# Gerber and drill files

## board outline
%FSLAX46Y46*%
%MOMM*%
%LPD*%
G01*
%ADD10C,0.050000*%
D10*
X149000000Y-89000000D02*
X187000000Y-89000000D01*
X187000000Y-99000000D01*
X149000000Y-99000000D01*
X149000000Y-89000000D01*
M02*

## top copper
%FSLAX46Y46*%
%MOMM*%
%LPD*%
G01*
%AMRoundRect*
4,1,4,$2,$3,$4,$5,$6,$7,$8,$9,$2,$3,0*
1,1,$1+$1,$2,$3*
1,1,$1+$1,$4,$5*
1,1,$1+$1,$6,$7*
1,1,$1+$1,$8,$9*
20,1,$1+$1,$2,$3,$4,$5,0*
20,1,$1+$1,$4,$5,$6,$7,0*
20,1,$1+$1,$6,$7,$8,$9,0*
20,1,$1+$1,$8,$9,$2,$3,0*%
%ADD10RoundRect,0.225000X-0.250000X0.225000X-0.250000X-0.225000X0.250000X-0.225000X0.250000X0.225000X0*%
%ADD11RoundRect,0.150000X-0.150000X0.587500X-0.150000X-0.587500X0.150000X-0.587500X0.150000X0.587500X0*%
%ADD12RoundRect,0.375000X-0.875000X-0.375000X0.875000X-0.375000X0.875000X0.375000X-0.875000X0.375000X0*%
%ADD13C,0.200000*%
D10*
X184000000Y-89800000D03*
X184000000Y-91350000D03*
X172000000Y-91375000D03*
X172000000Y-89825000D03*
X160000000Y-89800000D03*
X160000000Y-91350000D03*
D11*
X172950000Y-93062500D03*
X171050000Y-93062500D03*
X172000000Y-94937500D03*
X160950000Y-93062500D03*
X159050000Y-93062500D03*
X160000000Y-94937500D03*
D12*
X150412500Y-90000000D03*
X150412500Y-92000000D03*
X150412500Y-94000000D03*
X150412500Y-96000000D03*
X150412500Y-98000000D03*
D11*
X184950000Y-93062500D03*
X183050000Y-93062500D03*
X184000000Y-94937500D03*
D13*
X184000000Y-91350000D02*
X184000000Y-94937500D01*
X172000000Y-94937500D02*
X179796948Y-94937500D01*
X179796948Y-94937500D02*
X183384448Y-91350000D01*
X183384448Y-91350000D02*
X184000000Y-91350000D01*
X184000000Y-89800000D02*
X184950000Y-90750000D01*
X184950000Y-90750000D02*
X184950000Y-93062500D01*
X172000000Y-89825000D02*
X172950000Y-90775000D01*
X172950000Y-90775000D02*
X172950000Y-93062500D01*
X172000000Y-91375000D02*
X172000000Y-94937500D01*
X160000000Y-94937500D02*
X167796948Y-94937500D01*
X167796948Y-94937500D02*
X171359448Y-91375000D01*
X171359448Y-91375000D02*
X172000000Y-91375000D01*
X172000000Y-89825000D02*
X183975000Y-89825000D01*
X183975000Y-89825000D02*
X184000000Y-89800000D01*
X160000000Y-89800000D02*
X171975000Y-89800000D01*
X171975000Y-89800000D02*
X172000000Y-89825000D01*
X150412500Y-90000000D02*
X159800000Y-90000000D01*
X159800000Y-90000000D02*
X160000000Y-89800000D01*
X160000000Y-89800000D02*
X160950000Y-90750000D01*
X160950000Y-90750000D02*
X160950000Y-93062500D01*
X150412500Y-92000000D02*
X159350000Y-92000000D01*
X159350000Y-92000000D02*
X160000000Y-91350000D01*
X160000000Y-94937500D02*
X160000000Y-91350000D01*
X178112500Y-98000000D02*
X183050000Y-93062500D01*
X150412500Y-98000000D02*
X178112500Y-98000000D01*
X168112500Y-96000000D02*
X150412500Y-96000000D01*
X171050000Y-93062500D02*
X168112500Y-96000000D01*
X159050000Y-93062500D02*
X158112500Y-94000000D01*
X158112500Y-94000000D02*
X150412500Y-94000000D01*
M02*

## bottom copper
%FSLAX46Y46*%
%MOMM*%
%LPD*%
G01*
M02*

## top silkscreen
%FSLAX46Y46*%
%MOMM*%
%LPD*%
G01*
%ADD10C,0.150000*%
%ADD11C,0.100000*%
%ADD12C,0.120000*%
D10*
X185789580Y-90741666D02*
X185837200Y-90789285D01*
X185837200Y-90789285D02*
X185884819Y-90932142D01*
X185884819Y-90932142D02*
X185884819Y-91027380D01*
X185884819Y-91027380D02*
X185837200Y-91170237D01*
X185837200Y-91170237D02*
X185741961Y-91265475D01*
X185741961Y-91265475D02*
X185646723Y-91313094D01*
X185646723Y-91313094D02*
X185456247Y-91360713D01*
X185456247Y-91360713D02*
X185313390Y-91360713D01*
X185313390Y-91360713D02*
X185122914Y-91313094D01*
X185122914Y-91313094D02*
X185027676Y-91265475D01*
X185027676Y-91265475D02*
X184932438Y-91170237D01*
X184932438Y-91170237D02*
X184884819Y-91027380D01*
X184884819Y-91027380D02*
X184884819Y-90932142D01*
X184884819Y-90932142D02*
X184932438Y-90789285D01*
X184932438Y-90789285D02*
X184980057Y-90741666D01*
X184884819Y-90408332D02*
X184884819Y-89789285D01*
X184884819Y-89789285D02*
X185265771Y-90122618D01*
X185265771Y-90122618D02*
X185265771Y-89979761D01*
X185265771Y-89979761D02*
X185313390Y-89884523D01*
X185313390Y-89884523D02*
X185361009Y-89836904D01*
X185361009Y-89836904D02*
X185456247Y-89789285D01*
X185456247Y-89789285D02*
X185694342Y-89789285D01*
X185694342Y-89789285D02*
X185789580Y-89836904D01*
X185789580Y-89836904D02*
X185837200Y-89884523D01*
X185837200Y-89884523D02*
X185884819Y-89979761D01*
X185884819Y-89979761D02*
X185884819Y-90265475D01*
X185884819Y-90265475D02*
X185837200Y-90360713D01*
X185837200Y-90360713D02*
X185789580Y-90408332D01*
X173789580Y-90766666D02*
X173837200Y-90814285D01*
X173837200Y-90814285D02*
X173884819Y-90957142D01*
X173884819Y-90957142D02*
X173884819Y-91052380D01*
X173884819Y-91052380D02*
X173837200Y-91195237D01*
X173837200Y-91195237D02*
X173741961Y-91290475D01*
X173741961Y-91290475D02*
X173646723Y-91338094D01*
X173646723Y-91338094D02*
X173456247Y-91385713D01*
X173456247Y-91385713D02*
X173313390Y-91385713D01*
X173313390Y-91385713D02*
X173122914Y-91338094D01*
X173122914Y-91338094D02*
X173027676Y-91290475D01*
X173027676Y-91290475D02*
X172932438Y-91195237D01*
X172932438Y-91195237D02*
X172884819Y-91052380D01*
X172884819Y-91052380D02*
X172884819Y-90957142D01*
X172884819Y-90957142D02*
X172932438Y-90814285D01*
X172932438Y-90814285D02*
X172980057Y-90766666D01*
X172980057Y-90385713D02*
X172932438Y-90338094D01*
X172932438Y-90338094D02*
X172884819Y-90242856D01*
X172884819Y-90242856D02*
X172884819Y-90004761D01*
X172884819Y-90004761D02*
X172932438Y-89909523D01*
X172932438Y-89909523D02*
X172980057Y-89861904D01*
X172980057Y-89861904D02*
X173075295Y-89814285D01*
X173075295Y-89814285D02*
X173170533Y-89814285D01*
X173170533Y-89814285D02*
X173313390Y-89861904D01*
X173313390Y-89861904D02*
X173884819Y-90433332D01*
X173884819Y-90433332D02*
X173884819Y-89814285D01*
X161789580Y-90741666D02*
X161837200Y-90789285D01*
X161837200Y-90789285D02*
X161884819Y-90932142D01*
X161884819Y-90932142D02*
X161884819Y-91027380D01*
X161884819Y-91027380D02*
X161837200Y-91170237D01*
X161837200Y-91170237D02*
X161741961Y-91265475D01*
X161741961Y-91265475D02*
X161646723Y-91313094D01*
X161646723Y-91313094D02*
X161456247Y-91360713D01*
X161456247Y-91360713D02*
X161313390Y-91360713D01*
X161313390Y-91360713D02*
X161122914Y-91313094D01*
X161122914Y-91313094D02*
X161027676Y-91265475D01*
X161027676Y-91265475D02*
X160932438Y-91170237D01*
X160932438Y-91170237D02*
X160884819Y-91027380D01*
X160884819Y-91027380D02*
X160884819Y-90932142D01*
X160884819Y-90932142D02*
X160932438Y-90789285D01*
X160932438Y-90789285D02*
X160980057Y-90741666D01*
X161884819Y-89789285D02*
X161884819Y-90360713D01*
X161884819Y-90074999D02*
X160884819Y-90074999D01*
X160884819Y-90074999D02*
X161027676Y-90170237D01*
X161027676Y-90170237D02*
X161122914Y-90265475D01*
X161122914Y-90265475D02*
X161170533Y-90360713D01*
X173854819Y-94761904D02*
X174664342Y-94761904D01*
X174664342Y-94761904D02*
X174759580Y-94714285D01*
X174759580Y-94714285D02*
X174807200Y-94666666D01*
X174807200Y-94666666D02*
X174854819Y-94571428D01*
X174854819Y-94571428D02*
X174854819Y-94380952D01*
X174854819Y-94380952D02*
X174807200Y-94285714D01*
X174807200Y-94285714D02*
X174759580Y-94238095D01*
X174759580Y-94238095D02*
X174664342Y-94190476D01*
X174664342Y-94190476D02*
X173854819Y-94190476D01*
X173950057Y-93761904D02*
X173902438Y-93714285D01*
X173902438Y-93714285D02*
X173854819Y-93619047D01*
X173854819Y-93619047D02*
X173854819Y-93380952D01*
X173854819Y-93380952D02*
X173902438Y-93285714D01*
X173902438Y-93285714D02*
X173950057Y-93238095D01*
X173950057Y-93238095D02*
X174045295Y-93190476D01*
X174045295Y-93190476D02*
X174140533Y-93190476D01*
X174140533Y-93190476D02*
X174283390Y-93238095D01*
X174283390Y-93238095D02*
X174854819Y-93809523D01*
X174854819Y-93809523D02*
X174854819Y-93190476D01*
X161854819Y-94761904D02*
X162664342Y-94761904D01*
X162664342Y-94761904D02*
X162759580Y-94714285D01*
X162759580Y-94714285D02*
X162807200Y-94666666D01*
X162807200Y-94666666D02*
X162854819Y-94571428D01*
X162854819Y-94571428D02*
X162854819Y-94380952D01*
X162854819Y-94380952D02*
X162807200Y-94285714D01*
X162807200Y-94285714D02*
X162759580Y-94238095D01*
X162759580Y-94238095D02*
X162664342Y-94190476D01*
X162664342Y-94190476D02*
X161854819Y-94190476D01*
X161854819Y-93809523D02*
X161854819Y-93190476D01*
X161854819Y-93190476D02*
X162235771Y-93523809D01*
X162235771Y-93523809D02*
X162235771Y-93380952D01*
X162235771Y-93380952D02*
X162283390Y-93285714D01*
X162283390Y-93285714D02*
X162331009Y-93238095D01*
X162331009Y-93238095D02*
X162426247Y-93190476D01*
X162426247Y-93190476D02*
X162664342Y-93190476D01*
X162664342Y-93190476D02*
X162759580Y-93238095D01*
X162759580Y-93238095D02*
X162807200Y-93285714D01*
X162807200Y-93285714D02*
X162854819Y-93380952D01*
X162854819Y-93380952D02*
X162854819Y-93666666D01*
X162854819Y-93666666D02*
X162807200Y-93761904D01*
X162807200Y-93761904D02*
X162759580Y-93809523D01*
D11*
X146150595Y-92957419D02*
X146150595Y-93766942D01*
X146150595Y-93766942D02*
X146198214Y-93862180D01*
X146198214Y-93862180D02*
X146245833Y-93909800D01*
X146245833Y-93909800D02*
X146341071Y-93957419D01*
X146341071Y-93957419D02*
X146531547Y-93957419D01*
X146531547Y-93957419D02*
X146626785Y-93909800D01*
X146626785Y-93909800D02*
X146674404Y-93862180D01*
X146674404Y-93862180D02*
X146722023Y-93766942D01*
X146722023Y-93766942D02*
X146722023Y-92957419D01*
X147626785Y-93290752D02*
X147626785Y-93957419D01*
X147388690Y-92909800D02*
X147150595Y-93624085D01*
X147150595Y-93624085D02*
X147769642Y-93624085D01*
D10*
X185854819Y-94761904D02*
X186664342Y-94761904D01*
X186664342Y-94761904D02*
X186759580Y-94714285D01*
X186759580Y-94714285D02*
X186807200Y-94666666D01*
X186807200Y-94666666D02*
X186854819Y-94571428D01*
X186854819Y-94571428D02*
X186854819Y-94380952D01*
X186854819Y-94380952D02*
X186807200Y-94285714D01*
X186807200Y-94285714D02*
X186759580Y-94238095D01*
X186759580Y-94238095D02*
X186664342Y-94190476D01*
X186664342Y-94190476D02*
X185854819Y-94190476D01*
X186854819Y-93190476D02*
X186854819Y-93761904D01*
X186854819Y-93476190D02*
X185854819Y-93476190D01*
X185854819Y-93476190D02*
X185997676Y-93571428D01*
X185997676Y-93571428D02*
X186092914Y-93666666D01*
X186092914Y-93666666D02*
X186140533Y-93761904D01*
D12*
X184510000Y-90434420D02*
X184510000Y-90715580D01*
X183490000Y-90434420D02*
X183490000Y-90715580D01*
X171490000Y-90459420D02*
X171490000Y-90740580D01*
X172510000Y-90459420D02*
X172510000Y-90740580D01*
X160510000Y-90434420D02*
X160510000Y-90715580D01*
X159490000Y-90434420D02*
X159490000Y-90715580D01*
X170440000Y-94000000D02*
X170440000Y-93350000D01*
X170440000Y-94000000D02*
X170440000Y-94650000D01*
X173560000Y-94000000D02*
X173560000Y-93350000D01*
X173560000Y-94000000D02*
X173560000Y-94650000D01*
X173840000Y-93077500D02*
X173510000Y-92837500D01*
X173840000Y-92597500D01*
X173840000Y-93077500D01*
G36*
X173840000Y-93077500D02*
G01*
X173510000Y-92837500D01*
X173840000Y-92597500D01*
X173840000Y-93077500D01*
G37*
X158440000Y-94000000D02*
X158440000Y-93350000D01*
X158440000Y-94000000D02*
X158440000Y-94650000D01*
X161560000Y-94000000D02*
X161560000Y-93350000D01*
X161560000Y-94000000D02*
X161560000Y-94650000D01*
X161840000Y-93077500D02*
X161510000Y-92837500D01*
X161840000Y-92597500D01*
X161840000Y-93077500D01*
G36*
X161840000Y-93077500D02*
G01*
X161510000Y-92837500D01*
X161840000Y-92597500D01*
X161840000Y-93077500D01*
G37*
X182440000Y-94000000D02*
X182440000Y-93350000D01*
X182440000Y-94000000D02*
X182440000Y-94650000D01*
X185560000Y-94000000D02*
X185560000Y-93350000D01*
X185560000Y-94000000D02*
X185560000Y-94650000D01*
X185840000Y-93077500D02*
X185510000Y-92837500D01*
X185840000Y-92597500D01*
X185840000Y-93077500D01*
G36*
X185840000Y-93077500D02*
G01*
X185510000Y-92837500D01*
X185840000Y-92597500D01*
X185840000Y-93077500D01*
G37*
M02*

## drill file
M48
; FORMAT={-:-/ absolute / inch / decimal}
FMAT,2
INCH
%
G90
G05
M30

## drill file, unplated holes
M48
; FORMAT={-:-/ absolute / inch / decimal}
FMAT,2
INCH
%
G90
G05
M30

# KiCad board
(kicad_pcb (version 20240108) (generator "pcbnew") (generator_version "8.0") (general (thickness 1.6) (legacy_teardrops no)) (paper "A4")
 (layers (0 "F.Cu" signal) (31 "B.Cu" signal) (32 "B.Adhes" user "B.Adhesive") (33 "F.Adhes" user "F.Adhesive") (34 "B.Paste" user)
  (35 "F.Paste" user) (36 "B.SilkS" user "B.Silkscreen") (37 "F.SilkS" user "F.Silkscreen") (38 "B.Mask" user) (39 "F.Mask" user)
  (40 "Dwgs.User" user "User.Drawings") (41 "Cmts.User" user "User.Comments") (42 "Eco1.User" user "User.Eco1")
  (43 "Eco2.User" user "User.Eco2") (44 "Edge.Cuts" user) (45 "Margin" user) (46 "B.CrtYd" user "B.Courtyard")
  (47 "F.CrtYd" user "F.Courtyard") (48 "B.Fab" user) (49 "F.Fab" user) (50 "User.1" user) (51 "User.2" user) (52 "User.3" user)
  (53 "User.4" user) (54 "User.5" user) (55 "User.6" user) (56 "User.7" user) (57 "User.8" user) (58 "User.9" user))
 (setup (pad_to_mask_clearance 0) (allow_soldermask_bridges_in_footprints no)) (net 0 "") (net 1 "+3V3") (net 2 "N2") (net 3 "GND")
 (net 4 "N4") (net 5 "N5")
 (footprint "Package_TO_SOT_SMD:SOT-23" (layer "F.Cu") (at 172 94 -90)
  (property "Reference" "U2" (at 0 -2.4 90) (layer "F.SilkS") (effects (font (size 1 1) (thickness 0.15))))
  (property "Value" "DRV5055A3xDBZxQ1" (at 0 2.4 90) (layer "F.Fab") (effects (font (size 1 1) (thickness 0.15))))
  (fp_line (start 0 1.56) (end -0.65 1.56) (stroke (width 0.12) (type solid)) (layer "F.SilkS"))
  (fp_line (start 0 1.56) (end 0.65 1.56) (stroke (width 0.12) (type solid)) (layer "F.SilkS"))
  (fp_line (start 0 -1.56) (end -0.65 -1.56) (stroke (width 0.12) (type solid)) (layer "F.SilkS"))
  (fp_line (start 0 -1.56) (end 0.65 -1.56) (stroke (width 0.12) (type solid)) (layer "F.SilkS"))
  (fp_poly
   (pts (xy -1.1625 -1.51) (xy -1.4025 -1.84) (xy -0.9225 -1.84) (xy -1.1625 -1.51)) (stroke (width 0.12) (type solid)) (fill solid)
   (layer "F.SilkS"))
  (pad "1" smd roundrect (at -0.9375 -0.95 270) (size 1.475 0.6) (layers "F.Cu" "F.Paste" "F.Mask") (roundrect_rratio 0.25) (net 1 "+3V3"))
  (pad "2" smd roundrect (at -0.9375 0.95 270) (size 1.475 0.6) (layers "F.Cu" "F.Paste" "F.Mask") (roundrect_rratio 0.25) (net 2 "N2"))
  (pad "3" smd roundrect (at 0.9375 0 270) (size 1.475 0.6) (layers "F.Cu" "F.Paste" "F.Mask") (roundrect_rratio 0.25) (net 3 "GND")))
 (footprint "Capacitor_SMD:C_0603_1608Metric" (layer "F.Cu") (at 184 90.575 -90)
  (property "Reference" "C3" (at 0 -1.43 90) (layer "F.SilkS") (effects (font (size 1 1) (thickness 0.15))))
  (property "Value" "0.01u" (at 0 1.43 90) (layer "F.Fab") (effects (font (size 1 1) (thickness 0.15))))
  (fp_line (start -0.14058 0.51) (end 0.14058 0.51) (stroke (width 0.12) (type solid)) (layer "F.SilkS"))
  (fp_line (start -0.14058 -0.51) (end 0.14058 -0.51) (stroke (width 0.12) (type solid)) (layer "F.SilkS"))
  (pad "1" smd roundrect (at -0.775 0 270) (size 0.9 0.95) (layers "F.Cu" "F.Paste" "F.Mask") (roundrect_rratio 0.25) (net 1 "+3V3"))
  (pad "2" smd roundrect (at 0.775 0 270) (size 0.9 0.95) (layers "F.Cu" "F.Paste" "F.Mask") (roundrect_rratio 0.25) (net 3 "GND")))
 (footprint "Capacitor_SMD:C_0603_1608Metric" (layer "F.Cu") (at 160 90.575 -90)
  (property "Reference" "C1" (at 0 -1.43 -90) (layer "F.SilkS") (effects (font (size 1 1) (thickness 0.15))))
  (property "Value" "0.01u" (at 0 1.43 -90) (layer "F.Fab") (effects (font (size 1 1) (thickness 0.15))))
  (fp_line (start -0.14058 0.51) (end 0.14058 0.51) (stroke (width 0.12) (type solid)) (layer "F.SilkS"))
  (fp_line (start -0.14058 -0.51) (end 0.14058 -0.51) (stroke (width 0.12) (type solid)) (layer "F.SilkS"))
  (pad "1" smd roundrect (at -0.775 0 270) (size 0.9 0.95) (layers "F.Cu" "F.Paste" "F.Mask") (roundrect_rratio 0.25) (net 1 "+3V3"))
  (pad "2" smd roundrect (at 0.775 0 270) (size 0.9 0.95) (layers "F.Cu" "F.Paste" "F.Mask") (roundrect_rratio 0.25) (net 3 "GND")))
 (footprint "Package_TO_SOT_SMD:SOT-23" (layer "F.Cu") (at 160 94 -90)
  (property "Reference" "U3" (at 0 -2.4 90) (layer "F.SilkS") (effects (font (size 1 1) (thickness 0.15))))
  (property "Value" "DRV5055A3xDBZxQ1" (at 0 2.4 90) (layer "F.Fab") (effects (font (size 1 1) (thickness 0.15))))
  (fp_line (start 0 1.56) (end -0.65 1.56) (stroke (width 0.12) (type solid)) (layer "F.SilkS"))
  (fp_line (start 0 1.56) (end 0.65 1.56) (stroke (width 0.12) (type solid)) (layer "F.SilkS"))
  (fp_line (start 0 -1.56) (end -0.65 -1.56) (stroke (width 0.12) (type solid)) (layer "F.SilkS"))
  (fp_line (start 0 -1.56) (end 0.65 -1.56) (stroke (width 0.12) (type solid)) (layer "F.SilkS"))
  (fp_poly
   (pts (xy -1.1625 -1.51) (xy -1.4025 -1.84) (xy -0.9225 -1.84) (xy -1.1625 -1.51)) (stroke (width 0.12) (type solid)) (fill solid)
   (layer "F.SilkS"))
  (pad "1" smd roundrect (at -0.9375 -0.95 270) (size 1.475 0.6) (layers "F.Cu" "F.Paste" "F.Mask") (roundrect_rratio 0.25) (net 1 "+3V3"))
  (pad "2" smd roundrect (at -0.9375 0.95 270) (size 1.475 0.6) (layers "F.Cu" "F.Paste" "F.Mask") (roundrect_rratio 0.25) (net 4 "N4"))
  (pad "3" smd roundrect (at 0.9375 0 270) (size 1.475 0.6) (layers "F.Cu" "F.Paste" "F.Mask") (roundrect_rratio 0.25) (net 3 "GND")))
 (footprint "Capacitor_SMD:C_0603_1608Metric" (layer "F.Cu") (at 172 90.6 -90)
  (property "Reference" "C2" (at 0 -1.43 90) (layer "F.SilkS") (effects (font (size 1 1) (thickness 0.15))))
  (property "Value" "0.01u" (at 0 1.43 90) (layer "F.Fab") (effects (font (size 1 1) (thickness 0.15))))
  (fp_line (start -0.14058 0.51) (end 0.14058 0.51) (stroke (width 0.12) (type solid)) (layer "F.SilkS"))
  (fp_line (start -0.14058 -0.51) (end 0.14058 -0.51) (stroke (width 0.12) (type solid)) (layer "F.SilkS"))
  (pad "1" smd roundrect (at -0.775 0 270) (size 0.9 0.95) (layers "F.Cu" "F.Paste" "F.Mask") (roundrect_rratio 0.25) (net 1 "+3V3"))
  (pad "2" smd roundrect (at 0.775 0 270) (size 0.9 0.95) (layers "F.Cu" "F.Paste" "F.Mask") (roundrect_rratio 0.25) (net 3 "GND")))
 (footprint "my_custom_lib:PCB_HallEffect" (layer "F.Cu") (at 150.4125 94)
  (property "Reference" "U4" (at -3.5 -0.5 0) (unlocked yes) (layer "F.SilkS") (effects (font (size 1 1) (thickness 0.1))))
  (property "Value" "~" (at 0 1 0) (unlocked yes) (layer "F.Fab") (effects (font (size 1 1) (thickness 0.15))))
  (pad "1" smd roundrect (at 0 -4) (size 2.5 1.5) (layers "F.Cu" "F.Paste" "F.Mask") (roundrect_rratio 0.25) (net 1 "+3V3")
   (thermal_bridge_angle 45))
  (pad "2" smd roundrect (at 0 -2) (size 2.5 1.5) (layers "F.Cu" "F.Paste" "F.Mask") (roundrect_rratio 0.25) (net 3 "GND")
   (thermal_bridge_angle 45))
  (pad "3" smd roundrect (at 0 0) (size 2.5 1.5) (layers "F.Cu" "F.Paste" "F.Mask") (roundrect_rratio 0.25) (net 4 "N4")
   (thermal_bridge_angle 45))
  (pad "4" smd roundrect (at 0 2) (size 2.5 1.5) (layers "F.Cu" "F.Paste" "F.Mask") (roundrect_rratio 0.25) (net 2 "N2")
   (thermal_bridge_angle 45))
  (pad "5" smd roundrect (at 0 4) (size 2.5 1.5) (layers "F.Cu" "F.Paste" "F.Mask") (roundrect_rratio 0.25) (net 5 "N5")
   (thermal_bridge_angle 45)))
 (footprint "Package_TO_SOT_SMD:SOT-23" (layer "F.Cu") (at 184 94 -90)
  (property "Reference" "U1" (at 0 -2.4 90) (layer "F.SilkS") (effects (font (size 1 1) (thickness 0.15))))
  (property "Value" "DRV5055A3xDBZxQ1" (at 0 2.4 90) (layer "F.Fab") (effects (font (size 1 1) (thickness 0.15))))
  (fp_line (start 0 1.56) (end -0.65 1.56) (stroke (width 0.12) (type solid)) (layer "F.SilkS"))
  (fp_line (start 0 1.56) (end 0.65 1.56) (stroke (width 0.12) (type solid)) (layer "F.SilkS"))
  (fp_line (start 0 -1.56) (end -0.65 -1.56) (stroke (width 0.12) (type solid)) (layer "F.SilkS"))
  (fp_line (start 0 -1.56) (end 0.65 -1.56) (stroke (width 0.12) (type solid)) (layer "F.SilkS"))
  (fp_poly
   (pts (xy -1.1625 -1.51) (xy -1.4025 -1.84) (xy -0.9225 -1.84) (xy -1.1625 -1.51)) (stroke (width 0.12) (type solid)) (fill solid)
   (layer "F.SilkS"))
  (pad "1" smd roundrect (at -0.9375 -0.95 270) (size 1.475 0.6) (layers "F.Cu" "F.Paste" "F.Mask") (roundrect_rratio 0.25) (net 1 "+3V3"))
  (pad "2" smd roundrect (at -0.9375 0.95 270) (size 1.475 0.6) (layers "F.Cu" "F.Paste" "F.Mask") (roundrect_rratio 0.25) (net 5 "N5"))
  (pad "3" smd roundrect (at 0.9375 0 270) (size 1.475 0.6) (layers "F.Cu" "F.Paste" "F.Mask") (roundrect_rratio 0.25) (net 3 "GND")))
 (gr_rect (start 149 89) (end 187 99) (stroke (width 0.05) (type default)) (fill none) (layer "Edge.Cuts"))
 (segment (start 150.4125 92) (end 159.35 92) (width 0.2) (layer "F.Cu") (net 3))
 (segment (start 184 91.35) (end 184 94.9375) (width 0.2) (layer "F.Cu") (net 3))
 (segment (start 183.384448 91.35) (end 184 91.35) (width 0.2) (layer "F.Cu") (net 3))
 (segment (start 172 91.375) (end 172 94.9375) (width 0.2) (layer "F.Cu") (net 3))
 (segment (start 160 94.9375) (end 167.796948 94.9375) (width 0.2) (layer "F.Cu") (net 3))
 (segment (start 179.796948 94.9375) (end 183.384448 91.35) (width 0.2) (layer "F.Cu") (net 3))
 (segment (start 160 94.9375) (end 160 91.35) (width 0.2) (layer "F.Cu") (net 3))
 (segment (start 167.796948 94.9375) (end 171.359448 91.375) (width 0.2) (layer "F.Cu") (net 3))
 (segment (start 171.359448 91.375) (end 172 91.375) (width 0.2) (layer "F.Cu") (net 3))
 (segment (start 172 94.9375) (end 179.796948 94.9375) (width 0.2) (layer "F.Cu") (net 3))
 (segment (start 159.35 92) (end 160 91.35) (width 0.2) (layer "F.Cu") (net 3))
 (segment (start 184 89.8) (end 184.95 90.75) (width 0.2) (layer "F.Cu") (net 1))
 (segment (start 184.95 90.75) (end 184.95 93.0625) (width 0.2) (layer "F.Cu") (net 1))
 (segment (start 171.975 89.8) (end 172 89.825) (width 0.2) (layer "F.Cu") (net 1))
 (segment (start 160.95 90.75) (end 160.95 93.0625) (width 0.2) (layer "F.Cu") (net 1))
 (segment (start 160 89.8) (end 160.95 90.75) (width 0.2) (layer "F.Cu") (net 1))
 (segment (start 160 89.8) (end 171.975 89.8) (width 0.2) (layer "F.Cu") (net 1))
 (segment (start 159.8 90) (end 160 89.8) (width 0.2) (layer "F.Cu") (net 1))
 (segment (start 172 89.825) (end 183.975 89.825) (width 0.2) (layer "F.Cu") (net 1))
 (segment (start 172 89.825) (end 172.95 90.775) (width 0.2) (layer "F.Cu") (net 1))
 (segment (start 172.95 90.775) (end 172.95 93.0625) (width 0.2) (layer "F.Cu") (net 1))
 (segment (start 150.4125 90) (end 159.8 90) (width 0.2) (layer "F.Cu") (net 1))
 (segment (start 183.975 89.825) (end 184 89.8) (width 0.2) (layer "F.Cu") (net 1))
 (segment (start 178.1125 98) (end 183.05 93.0625) (width 0.2) (layer "F.Cu") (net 5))
 (segment (start 150.4125 98) (end 178.1125 98) (width 0.2) (layer "F.Cu") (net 5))
 (segment (start 168.1125 96) (end 150.4125 96) (width 0.2) (layer "F.Cu") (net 2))
 (segment (start 171.05 93.0625) (end 168.1125 96) (width 0.2) (layer "F.Cu") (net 2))
 (segment (start 159.05 93.0625) (end 158.1125 94) (width 0.2) (layer "F.Cu") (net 4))
 (segment (start 158.1125 94) (end 150.4125 94) (width 0.2) (layer "F.Cu") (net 4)))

